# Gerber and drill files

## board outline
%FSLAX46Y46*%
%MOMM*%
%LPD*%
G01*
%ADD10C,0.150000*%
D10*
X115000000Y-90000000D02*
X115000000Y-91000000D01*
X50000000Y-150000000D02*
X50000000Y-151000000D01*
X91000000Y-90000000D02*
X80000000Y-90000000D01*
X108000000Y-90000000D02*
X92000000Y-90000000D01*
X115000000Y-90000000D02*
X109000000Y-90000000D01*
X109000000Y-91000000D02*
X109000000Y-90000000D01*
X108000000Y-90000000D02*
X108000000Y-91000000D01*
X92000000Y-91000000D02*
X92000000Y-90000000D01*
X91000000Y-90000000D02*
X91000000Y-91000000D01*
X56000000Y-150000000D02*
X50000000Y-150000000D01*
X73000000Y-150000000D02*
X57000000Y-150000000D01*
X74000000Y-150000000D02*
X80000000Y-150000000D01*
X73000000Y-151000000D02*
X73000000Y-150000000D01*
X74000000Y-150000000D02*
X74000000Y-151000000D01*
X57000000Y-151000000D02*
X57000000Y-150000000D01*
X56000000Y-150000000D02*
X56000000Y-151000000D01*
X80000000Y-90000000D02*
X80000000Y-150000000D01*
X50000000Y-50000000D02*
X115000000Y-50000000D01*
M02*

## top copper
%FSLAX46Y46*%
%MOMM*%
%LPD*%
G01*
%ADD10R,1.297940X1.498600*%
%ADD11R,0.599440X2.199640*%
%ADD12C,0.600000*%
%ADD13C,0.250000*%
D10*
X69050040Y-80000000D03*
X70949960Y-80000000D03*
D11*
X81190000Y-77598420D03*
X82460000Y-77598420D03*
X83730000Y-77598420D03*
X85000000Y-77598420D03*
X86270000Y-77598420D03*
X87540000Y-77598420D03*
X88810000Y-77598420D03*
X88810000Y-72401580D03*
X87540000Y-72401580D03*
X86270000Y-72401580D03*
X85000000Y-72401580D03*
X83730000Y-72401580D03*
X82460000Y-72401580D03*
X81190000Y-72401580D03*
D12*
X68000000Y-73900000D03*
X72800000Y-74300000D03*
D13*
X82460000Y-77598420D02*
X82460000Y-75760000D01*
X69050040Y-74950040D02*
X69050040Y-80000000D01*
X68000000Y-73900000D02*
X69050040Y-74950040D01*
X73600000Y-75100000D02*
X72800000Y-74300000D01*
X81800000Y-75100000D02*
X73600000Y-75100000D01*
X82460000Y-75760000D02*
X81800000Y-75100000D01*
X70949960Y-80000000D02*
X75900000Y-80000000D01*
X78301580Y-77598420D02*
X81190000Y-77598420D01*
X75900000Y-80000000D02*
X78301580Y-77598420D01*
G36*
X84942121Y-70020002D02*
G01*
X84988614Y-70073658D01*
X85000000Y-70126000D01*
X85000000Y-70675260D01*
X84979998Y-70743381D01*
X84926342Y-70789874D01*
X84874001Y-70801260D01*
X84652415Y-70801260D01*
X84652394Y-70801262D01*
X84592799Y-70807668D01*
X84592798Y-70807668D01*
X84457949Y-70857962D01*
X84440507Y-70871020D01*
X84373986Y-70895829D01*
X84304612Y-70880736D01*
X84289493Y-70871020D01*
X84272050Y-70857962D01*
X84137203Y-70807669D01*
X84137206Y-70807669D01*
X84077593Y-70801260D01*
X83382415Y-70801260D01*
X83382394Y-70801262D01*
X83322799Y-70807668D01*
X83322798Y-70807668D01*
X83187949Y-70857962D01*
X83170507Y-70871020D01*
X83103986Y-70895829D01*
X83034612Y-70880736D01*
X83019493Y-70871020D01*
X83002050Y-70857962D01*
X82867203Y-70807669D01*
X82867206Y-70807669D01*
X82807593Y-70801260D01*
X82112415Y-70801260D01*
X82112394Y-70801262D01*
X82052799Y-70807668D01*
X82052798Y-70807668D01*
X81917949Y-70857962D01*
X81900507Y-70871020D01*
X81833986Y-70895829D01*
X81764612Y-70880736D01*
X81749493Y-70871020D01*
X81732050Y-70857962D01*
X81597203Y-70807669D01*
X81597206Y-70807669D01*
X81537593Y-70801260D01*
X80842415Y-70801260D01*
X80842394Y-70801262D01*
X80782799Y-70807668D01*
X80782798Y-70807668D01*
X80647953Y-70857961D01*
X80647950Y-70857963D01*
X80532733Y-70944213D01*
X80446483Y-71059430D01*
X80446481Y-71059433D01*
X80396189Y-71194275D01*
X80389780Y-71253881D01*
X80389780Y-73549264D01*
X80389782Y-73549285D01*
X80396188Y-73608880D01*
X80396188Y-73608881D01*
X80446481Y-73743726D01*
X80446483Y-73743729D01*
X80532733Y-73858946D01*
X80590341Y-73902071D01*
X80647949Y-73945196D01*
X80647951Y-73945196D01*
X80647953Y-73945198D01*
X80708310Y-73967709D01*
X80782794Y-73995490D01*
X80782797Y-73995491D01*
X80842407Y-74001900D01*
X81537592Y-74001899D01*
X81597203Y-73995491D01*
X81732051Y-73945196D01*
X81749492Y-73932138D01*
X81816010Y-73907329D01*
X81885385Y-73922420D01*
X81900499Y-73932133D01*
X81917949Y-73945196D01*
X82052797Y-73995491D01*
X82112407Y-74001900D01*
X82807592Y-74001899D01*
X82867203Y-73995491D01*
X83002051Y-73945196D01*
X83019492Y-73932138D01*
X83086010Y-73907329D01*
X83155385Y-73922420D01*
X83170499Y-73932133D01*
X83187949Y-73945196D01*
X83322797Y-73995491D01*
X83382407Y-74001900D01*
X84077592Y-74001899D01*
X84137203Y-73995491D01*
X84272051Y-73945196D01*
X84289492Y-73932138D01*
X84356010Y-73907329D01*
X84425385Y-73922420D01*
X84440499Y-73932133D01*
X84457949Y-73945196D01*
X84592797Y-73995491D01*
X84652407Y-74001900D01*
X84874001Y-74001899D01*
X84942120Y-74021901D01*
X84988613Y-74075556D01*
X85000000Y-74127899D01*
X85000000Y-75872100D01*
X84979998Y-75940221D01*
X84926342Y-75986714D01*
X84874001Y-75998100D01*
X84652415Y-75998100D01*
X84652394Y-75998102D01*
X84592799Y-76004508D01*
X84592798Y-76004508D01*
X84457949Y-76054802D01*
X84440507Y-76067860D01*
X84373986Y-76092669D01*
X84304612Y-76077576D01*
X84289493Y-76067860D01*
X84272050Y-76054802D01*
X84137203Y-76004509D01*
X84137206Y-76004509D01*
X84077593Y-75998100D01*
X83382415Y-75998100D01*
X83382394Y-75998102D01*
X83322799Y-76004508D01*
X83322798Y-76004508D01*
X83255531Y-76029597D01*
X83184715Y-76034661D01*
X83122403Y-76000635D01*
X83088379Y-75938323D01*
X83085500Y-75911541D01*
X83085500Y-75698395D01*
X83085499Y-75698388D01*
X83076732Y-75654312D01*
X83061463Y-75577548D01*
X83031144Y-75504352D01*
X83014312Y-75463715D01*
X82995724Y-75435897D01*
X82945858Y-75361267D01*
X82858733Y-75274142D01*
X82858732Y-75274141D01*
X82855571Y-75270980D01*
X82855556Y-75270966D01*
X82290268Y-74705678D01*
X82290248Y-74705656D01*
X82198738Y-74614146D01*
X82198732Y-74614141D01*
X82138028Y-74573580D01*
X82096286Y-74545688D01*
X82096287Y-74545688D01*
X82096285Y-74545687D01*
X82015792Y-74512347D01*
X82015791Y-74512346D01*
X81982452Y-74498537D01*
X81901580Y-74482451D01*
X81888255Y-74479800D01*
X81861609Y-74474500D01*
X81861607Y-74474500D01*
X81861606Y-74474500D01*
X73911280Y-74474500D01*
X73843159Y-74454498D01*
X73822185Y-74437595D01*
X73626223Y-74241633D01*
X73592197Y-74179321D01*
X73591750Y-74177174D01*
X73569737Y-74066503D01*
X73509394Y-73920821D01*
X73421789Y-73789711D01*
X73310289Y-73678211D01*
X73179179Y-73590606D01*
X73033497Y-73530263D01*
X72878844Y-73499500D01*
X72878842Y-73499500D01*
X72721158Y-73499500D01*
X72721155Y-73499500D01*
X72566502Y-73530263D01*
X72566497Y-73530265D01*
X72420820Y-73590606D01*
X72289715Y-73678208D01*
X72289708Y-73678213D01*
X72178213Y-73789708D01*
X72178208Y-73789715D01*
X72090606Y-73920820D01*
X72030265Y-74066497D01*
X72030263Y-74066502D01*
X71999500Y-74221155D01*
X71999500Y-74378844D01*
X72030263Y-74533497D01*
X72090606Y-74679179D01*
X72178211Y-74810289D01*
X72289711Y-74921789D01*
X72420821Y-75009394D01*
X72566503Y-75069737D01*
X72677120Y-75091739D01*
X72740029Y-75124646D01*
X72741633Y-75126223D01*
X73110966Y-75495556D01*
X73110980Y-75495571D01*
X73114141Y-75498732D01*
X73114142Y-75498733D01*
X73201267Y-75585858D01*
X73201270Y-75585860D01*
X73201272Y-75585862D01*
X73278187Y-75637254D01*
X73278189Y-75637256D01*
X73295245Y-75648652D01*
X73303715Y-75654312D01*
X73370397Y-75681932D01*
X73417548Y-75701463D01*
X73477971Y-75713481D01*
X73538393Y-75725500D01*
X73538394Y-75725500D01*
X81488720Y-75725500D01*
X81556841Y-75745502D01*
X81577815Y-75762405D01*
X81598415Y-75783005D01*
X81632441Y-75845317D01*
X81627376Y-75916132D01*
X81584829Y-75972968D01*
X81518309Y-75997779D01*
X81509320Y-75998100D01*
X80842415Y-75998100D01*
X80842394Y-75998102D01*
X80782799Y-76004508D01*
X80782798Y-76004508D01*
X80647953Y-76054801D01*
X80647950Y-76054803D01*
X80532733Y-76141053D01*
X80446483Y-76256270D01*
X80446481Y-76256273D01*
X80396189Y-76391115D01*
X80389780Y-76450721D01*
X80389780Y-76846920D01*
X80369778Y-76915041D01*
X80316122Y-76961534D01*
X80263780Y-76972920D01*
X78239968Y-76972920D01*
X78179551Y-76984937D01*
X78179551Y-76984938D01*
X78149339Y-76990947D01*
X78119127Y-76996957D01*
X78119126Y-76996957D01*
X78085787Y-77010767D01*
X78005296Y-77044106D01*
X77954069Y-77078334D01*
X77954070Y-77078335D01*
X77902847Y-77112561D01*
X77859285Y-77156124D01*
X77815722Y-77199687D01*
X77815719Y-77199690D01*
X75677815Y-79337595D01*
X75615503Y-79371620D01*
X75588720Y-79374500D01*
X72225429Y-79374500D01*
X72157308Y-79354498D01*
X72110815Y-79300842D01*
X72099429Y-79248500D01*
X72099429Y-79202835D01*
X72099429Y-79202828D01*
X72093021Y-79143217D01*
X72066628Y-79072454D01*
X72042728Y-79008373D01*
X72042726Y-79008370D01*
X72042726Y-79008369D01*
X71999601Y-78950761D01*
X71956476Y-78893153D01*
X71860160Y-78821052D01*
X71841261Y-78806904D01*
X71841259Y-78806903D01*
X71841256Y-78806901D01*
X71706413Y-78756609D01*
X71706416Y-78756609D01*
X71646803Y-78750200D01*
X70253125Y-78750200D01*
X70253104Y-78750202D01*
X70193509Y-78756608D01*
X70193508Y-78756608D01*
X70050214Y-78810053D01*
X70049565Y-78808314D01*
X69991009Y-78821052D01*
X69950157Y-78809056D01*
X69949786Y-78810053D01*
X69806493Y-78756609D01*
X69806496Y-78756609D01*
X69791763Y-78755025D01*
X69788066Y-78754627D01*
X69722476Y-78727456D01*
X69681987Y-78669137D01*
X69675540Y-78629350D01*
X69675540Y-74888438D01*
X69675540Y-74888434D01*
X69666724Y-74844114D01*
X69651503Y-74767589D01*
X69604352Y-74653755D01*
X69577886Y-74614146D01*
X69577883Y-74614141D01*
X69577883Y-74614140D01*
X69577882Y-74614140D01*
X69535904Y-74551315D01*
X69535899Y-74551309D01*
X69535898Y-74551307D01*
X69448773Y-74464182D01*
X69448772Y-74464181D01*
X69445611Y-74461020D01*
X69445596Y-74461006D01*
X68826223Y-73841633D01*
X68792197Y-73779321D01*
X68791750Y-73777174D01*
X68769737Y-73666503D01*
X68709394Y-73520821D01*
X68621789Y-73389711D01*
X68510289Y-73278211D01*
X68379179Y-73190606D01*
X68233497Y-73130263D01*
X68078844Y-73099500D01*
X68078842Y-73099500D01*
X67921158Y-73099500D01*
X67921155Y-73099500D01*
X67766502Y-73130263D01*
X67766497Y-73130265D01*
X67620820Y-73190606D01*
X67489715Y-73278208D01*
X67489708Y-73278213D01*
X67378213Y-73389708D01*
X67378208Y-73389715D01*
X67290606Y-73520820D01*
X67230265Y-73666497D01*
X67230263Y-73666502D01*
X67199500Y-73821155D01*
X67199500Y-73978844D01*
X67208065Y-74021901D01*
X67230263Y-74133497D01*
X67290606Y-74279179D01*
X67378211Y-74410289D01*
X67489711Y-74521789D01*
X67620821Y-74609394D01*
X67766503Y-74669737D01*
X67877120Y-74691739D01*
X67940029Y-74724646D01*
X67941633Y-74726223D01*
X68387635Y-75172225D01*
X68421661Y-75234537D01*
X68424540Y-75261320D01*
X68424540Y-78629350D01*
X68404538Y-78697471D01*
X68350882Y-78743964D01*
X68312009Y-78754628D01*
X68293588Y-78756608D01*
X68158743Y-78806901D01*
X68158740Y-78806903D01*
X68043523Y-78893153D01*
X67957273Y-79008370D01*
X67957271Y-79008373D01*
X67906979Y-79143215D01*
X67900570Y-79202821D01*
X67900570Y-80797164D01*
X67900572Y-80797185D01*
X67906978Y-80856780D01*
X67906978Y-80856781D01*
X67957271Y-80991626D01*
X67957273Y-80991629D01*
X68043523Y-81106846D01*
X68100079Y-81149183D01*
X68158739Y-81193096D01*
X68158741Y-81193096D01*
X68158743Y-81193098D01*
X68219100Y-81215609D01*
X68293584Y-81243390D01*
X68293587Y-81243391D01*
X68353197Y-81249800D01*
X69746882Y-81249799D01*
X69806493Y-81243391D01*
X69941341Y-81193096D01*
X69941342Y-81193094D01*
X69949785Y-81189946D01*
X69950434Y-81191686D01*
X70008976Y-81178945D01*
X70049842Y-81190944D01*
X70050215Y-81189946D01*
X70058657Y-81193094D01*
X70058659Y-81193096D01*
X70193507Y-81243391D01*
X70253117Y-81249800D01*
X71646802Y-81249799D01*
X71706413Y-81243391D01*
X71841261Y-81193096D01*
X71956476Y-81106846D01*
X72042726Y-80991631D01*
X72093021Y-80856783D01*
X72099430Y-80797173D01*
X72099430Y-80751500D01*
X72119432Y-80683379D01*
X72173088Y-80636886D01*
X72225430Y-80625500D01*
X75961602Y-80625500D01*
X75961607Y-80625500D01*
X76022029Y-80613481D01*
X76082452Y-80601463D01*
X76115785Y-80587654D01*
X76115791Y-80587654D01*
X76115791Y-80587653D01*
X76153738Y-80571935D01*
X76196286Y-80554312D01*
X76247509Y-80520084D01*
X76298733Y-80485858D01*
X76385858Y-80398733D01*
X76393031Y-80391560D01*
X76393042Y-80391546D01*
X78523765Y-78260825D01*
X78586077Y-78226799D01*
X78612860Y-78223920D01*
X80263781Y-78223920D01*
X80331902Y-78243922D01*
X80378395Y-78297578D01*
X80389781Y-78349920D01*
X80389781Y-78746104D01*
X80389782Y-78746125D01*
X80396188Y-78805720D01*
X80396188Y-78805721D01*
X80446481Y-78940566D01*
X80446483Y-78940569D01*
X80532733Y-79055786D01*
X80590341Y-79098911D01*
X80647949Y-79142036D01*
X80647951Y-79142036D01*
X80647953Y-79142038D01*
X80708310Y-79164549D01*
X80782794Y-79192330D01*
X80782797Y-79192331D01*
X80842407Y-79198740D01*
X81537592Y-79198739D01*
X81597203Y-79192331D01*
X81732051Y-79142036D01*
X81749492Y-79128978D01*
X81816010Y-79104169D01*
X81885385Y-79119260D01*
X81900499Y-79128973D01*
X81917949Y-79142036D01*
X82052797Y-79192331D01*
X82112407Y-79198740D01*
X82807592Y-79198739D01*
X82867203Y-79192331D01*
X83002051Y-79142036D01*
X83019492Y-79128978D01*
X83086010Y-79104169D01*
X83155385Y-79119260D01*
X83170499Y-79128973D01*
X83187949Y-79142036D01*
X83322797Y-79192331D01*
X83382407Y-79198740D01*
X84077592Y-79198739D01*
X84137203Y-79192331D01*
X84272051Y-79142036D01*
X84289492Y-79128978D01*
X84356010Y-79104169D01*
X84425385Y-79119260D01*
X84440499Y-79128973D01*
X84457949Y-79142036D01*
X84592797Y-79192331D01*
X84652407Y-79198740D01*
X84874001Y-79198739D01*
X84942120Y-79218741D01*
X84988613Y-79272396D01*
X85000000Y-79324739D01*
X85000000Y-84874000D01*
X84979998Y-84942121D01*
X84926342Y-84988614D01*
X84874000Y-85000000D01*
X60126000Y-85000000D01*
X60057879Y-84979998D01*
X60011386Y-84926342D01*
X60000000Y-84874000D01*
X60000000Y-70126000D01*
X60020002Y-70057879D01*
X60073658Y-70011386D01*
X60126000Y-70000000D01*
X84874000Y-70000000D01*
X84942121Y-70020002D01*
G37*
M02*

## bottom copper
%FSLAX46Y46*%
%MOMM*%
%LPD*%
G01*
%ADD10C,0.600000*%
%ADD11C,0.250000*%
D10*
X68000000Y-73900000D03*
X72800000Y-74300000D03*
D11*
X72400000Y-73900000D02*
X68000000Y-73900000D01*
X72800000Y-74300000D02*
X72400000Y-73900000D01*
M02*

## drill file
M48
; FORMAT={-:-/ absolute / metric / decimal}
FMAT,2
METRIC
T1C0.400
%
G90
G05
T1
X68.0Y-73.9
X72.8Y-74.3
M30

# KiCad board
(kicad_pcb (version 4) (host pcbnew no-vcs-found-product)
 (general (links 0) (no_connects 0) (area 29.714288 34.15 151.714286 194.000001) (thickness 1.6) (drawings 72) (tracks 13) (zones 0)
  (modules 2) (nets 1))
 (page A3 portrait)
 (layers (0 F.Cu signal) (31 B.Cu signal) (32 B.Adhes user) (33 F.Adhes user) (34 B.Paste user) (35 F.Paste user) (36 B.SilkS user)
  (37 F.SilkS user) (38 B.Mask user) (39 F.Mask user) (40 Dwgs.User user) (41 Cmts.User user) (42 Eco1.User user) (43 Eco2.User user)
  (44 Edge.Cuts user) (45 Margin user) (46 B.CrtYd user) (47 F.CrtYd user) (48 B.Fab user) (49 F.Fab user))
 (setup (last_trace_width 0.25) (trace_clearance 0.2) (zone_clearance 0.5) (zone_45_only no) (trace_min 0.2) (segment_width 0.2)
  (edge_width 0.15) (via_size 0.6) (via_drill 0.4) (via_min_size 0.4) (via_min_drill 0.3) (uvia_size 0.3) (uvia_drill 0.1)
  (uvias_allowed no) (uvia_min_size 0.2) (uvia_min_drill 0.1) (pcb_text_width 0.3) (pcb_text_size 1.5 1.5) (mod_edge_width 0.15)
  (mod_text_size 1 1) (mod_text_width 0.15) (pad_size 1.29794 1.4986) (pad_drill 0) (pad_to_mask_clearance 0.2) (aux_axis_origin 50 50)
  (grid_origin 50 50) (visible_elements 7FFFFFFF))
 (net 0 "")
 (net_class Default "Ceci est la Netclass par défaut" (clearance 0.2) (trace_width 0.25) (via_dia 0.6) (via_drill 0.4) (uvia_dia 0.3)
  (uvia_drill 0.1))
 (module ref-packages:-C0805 (layer F.Cu) (at 70 80)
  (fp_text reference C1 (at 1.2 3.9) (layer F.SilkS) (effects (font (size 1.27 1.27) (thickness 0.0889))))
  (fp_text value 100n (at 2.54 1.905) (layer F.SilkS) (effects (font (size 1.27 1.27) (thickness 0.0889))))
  (pad 1 smd rect (at -0.94996 0) (size 1.29794 1.4986) (layers F.Cu F.Paste F.Mask))
  (pad 2 smd rect (at 0.94996 0) (size 1.29794 1.4986) (layers F.Cu F.Paste F.Mask)))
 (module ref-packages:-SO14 (layer F.Cu) (at 85 75)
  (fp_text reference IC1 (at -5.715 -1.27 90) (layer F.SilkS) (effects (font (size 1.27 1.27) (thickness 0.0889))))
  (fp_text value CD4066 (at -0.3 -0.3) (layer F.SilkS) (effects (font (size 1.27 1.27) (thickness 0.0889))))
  (pad 1 smd rect (at -3.81 2.59842) (size 0.59944 2.19964) (layers F.Cu F.Paste F.Mask))
  (pad 2 smd rect (at -2.54 2.59842) (size 0.59944 2.19964) (layers F.Cu F.Paste F.Mask))
  (pad 3 smd rect (at -1.27 2.59842) (size 0.59944 2.19964) (layers F.Cu F.Paste F.Mask))
  (pad 4 smd rect (at 0 2.59842) (size 0.59944 2.19964) (layers F.Cu F.Paste F.Mask))
  (pad 5 smd rect (at 1.27 2.59842) (size 0.59944 2.19964) (layers F.Cu F.Paste F.Mask))
  (pad 6 smd rect (at 2.54 2.59842) (size 0.59944 2.19964) (layers F.Cu F.Paste F.Mask))
  (pad 7 smd rect (at 3.81 2.59842) (size 0.59944 2.19964) (layers F.Cu F.Paste F.Mask))
  (pad 8 smd rect (at 3.81 -2.59842) (size 0.59944 2.19964) (layers F.Cu F.Paste F.Mask))
  (pad 9 smd rect (at 2.54 -2.59842) (size 0.59944 2.19964) (layers F.Cu F.Paste F.Mask))
  (pad 10 smd rect (at 1.27 -2.59842) (size 0.59944 2.19964) (layers F.Cu F.Paste F.Mask))
  (pad 11 smd rect (at 0 -2.59842) (size 0.59944 2.19964) (layers F.Cu F.Paste F.Mask))
  (pad 12 smd rect (at -1.27 -2.59842) (size 0.59944 2.19964) (layers F.Cu F.Paste F.Mask))
  (pad 13 smd rect (at -2.54 -2.59842) (size 0.59944 2.19964) (layers F.Cu F.Paste F.Mask))
  (pad 14 smd rect (at -3.81 -2.59842) (size 0.59944 2.19964) (layers F.Cu F.Paste F.Mask)))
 (gr_line (start 115 90) (end 115 91) (angle 90) (layer Edge.Cuts) (width 0.15))
 (gr_line (start 50 150) (end 50 151) (angle 90) (layer Edge.Cuts) (width 0.15))
 (gr_line (start 91 90) (end 80 90) (angle 90) (layer Edge.Cuts) (width 0.15))
 (gr_line (start 108 90) (end 92 90) (angle 90) (layer Edge.Cuts) (width 0.15))
 (gr_line (start 115 90) (end 109 90) (angle 90) (layer Edge.Cuts) (width 0.15))
 (gr_line (start 109 91) (end 109 90) (angle 90) (layer Edge.Cuts) (width 0.15))
 (gr_line (start 108 90) (end 108 91) (angle 90) (layer Edge.Cuts) (width 0.15))
 (gr_line (start 92 91) (end 92 90) (angle 90) (layer Edge.Cuts) (width 0.15))
 (gr_line (start 91 90) (end 91 91) (angle 90) (layer Edge.Cuts) (width 0.15))
 (gr_line (start 56 150) (end 50 150) (angle 90) (layer Edge.Cuts) (width 0.15))
 (gr_line (start 73 150) (end 57 150) (angle 90) (layer Edge.Cuts) (width 0.15))
 (gr_line (start 74 150) (end 80 150) (angle 90) (layer Edge.Cuts) (width 0.15))
 (gr_line (start 73 151) (end 73 150) (angle 90) (layer Edge.Cuts) (width 0.15))
 (gr_line (start 74 150) (end 74 151) (angle 90) (layer Edge.Cuts) (width 0.15))
 (gr_line (start 57 151) (end 57 150) (angle 90) (layer Edge.Cuts) (width 0.15))
 (gr_line (start 56 150) (end 56 151) (angle 90) (layer Edge.Cuts) (width 0.15))
 (gr_line (start 80 90) (end 80 150) (angle 90) (layer Edge.Cuts) (width 0.15))
 (gr_line (start 50 50) (end 115 50) (angle 90) (layer Edge.Cuts) (width 0.15))
 (segment (start 82.46 77.59842) (end 82.46 75.76) (width 0.25) (layer F.Cu) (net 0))
 (segment (start 69.05004 74.95004) (end 69.05004 80) (width 0.25) (layer F.Cu) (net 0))
 (segment (start 68 73.9) (end 69.05004 74.95004) (width 0.25) (layer F.Cu) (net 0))
 (via (at 68 73.9) (size 0.6) (drill 0.4) (layers F.Cu B.Cu) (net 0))
 (segment (start 72.4 73.9) (end 68 73.9) (width 0.25) (layer B.Cu) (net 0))
 (segment (start 72.8 74.3) (end 72.4 73.9) (width 0.25) (layer B.Cu) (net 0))
 (via (at 72.8 74.3) (size 0.6) (drill 0.4) (layers F.Cu B.Cu) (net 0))
 (segment (start 73.6 75.1) (end 72.8 74.3) (width 0.25) (layer F.Cu) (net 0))
 (segment (start 81.8 75.1) (end 73.6 75.1) (width 0.25) (layer F.Cu) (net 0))
 (segment (start 82.46 75.76) (end 81.8 75.1) (width 0.25) (layer F.Cu) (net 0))
 (segment (start 70.94996 80) (end 75.9 80) (width 0.25) (layer F.Cu) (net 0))
 (segment (start 78.30158 77.59842) (end 81.19 77.59842) (width 0.25) (layer F.Cu) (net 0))
 (segment (start 75.9 80) (end 78.30158 77.59842) (width 0.25) (layer F.Cu) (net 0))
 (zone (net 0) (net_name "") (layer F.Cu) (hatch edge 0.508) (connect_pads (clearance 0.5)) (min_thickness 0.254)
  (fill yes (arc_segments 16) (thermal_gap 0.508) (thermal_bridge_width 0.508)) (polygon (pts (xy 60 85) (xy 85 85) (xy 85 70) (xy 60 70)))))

